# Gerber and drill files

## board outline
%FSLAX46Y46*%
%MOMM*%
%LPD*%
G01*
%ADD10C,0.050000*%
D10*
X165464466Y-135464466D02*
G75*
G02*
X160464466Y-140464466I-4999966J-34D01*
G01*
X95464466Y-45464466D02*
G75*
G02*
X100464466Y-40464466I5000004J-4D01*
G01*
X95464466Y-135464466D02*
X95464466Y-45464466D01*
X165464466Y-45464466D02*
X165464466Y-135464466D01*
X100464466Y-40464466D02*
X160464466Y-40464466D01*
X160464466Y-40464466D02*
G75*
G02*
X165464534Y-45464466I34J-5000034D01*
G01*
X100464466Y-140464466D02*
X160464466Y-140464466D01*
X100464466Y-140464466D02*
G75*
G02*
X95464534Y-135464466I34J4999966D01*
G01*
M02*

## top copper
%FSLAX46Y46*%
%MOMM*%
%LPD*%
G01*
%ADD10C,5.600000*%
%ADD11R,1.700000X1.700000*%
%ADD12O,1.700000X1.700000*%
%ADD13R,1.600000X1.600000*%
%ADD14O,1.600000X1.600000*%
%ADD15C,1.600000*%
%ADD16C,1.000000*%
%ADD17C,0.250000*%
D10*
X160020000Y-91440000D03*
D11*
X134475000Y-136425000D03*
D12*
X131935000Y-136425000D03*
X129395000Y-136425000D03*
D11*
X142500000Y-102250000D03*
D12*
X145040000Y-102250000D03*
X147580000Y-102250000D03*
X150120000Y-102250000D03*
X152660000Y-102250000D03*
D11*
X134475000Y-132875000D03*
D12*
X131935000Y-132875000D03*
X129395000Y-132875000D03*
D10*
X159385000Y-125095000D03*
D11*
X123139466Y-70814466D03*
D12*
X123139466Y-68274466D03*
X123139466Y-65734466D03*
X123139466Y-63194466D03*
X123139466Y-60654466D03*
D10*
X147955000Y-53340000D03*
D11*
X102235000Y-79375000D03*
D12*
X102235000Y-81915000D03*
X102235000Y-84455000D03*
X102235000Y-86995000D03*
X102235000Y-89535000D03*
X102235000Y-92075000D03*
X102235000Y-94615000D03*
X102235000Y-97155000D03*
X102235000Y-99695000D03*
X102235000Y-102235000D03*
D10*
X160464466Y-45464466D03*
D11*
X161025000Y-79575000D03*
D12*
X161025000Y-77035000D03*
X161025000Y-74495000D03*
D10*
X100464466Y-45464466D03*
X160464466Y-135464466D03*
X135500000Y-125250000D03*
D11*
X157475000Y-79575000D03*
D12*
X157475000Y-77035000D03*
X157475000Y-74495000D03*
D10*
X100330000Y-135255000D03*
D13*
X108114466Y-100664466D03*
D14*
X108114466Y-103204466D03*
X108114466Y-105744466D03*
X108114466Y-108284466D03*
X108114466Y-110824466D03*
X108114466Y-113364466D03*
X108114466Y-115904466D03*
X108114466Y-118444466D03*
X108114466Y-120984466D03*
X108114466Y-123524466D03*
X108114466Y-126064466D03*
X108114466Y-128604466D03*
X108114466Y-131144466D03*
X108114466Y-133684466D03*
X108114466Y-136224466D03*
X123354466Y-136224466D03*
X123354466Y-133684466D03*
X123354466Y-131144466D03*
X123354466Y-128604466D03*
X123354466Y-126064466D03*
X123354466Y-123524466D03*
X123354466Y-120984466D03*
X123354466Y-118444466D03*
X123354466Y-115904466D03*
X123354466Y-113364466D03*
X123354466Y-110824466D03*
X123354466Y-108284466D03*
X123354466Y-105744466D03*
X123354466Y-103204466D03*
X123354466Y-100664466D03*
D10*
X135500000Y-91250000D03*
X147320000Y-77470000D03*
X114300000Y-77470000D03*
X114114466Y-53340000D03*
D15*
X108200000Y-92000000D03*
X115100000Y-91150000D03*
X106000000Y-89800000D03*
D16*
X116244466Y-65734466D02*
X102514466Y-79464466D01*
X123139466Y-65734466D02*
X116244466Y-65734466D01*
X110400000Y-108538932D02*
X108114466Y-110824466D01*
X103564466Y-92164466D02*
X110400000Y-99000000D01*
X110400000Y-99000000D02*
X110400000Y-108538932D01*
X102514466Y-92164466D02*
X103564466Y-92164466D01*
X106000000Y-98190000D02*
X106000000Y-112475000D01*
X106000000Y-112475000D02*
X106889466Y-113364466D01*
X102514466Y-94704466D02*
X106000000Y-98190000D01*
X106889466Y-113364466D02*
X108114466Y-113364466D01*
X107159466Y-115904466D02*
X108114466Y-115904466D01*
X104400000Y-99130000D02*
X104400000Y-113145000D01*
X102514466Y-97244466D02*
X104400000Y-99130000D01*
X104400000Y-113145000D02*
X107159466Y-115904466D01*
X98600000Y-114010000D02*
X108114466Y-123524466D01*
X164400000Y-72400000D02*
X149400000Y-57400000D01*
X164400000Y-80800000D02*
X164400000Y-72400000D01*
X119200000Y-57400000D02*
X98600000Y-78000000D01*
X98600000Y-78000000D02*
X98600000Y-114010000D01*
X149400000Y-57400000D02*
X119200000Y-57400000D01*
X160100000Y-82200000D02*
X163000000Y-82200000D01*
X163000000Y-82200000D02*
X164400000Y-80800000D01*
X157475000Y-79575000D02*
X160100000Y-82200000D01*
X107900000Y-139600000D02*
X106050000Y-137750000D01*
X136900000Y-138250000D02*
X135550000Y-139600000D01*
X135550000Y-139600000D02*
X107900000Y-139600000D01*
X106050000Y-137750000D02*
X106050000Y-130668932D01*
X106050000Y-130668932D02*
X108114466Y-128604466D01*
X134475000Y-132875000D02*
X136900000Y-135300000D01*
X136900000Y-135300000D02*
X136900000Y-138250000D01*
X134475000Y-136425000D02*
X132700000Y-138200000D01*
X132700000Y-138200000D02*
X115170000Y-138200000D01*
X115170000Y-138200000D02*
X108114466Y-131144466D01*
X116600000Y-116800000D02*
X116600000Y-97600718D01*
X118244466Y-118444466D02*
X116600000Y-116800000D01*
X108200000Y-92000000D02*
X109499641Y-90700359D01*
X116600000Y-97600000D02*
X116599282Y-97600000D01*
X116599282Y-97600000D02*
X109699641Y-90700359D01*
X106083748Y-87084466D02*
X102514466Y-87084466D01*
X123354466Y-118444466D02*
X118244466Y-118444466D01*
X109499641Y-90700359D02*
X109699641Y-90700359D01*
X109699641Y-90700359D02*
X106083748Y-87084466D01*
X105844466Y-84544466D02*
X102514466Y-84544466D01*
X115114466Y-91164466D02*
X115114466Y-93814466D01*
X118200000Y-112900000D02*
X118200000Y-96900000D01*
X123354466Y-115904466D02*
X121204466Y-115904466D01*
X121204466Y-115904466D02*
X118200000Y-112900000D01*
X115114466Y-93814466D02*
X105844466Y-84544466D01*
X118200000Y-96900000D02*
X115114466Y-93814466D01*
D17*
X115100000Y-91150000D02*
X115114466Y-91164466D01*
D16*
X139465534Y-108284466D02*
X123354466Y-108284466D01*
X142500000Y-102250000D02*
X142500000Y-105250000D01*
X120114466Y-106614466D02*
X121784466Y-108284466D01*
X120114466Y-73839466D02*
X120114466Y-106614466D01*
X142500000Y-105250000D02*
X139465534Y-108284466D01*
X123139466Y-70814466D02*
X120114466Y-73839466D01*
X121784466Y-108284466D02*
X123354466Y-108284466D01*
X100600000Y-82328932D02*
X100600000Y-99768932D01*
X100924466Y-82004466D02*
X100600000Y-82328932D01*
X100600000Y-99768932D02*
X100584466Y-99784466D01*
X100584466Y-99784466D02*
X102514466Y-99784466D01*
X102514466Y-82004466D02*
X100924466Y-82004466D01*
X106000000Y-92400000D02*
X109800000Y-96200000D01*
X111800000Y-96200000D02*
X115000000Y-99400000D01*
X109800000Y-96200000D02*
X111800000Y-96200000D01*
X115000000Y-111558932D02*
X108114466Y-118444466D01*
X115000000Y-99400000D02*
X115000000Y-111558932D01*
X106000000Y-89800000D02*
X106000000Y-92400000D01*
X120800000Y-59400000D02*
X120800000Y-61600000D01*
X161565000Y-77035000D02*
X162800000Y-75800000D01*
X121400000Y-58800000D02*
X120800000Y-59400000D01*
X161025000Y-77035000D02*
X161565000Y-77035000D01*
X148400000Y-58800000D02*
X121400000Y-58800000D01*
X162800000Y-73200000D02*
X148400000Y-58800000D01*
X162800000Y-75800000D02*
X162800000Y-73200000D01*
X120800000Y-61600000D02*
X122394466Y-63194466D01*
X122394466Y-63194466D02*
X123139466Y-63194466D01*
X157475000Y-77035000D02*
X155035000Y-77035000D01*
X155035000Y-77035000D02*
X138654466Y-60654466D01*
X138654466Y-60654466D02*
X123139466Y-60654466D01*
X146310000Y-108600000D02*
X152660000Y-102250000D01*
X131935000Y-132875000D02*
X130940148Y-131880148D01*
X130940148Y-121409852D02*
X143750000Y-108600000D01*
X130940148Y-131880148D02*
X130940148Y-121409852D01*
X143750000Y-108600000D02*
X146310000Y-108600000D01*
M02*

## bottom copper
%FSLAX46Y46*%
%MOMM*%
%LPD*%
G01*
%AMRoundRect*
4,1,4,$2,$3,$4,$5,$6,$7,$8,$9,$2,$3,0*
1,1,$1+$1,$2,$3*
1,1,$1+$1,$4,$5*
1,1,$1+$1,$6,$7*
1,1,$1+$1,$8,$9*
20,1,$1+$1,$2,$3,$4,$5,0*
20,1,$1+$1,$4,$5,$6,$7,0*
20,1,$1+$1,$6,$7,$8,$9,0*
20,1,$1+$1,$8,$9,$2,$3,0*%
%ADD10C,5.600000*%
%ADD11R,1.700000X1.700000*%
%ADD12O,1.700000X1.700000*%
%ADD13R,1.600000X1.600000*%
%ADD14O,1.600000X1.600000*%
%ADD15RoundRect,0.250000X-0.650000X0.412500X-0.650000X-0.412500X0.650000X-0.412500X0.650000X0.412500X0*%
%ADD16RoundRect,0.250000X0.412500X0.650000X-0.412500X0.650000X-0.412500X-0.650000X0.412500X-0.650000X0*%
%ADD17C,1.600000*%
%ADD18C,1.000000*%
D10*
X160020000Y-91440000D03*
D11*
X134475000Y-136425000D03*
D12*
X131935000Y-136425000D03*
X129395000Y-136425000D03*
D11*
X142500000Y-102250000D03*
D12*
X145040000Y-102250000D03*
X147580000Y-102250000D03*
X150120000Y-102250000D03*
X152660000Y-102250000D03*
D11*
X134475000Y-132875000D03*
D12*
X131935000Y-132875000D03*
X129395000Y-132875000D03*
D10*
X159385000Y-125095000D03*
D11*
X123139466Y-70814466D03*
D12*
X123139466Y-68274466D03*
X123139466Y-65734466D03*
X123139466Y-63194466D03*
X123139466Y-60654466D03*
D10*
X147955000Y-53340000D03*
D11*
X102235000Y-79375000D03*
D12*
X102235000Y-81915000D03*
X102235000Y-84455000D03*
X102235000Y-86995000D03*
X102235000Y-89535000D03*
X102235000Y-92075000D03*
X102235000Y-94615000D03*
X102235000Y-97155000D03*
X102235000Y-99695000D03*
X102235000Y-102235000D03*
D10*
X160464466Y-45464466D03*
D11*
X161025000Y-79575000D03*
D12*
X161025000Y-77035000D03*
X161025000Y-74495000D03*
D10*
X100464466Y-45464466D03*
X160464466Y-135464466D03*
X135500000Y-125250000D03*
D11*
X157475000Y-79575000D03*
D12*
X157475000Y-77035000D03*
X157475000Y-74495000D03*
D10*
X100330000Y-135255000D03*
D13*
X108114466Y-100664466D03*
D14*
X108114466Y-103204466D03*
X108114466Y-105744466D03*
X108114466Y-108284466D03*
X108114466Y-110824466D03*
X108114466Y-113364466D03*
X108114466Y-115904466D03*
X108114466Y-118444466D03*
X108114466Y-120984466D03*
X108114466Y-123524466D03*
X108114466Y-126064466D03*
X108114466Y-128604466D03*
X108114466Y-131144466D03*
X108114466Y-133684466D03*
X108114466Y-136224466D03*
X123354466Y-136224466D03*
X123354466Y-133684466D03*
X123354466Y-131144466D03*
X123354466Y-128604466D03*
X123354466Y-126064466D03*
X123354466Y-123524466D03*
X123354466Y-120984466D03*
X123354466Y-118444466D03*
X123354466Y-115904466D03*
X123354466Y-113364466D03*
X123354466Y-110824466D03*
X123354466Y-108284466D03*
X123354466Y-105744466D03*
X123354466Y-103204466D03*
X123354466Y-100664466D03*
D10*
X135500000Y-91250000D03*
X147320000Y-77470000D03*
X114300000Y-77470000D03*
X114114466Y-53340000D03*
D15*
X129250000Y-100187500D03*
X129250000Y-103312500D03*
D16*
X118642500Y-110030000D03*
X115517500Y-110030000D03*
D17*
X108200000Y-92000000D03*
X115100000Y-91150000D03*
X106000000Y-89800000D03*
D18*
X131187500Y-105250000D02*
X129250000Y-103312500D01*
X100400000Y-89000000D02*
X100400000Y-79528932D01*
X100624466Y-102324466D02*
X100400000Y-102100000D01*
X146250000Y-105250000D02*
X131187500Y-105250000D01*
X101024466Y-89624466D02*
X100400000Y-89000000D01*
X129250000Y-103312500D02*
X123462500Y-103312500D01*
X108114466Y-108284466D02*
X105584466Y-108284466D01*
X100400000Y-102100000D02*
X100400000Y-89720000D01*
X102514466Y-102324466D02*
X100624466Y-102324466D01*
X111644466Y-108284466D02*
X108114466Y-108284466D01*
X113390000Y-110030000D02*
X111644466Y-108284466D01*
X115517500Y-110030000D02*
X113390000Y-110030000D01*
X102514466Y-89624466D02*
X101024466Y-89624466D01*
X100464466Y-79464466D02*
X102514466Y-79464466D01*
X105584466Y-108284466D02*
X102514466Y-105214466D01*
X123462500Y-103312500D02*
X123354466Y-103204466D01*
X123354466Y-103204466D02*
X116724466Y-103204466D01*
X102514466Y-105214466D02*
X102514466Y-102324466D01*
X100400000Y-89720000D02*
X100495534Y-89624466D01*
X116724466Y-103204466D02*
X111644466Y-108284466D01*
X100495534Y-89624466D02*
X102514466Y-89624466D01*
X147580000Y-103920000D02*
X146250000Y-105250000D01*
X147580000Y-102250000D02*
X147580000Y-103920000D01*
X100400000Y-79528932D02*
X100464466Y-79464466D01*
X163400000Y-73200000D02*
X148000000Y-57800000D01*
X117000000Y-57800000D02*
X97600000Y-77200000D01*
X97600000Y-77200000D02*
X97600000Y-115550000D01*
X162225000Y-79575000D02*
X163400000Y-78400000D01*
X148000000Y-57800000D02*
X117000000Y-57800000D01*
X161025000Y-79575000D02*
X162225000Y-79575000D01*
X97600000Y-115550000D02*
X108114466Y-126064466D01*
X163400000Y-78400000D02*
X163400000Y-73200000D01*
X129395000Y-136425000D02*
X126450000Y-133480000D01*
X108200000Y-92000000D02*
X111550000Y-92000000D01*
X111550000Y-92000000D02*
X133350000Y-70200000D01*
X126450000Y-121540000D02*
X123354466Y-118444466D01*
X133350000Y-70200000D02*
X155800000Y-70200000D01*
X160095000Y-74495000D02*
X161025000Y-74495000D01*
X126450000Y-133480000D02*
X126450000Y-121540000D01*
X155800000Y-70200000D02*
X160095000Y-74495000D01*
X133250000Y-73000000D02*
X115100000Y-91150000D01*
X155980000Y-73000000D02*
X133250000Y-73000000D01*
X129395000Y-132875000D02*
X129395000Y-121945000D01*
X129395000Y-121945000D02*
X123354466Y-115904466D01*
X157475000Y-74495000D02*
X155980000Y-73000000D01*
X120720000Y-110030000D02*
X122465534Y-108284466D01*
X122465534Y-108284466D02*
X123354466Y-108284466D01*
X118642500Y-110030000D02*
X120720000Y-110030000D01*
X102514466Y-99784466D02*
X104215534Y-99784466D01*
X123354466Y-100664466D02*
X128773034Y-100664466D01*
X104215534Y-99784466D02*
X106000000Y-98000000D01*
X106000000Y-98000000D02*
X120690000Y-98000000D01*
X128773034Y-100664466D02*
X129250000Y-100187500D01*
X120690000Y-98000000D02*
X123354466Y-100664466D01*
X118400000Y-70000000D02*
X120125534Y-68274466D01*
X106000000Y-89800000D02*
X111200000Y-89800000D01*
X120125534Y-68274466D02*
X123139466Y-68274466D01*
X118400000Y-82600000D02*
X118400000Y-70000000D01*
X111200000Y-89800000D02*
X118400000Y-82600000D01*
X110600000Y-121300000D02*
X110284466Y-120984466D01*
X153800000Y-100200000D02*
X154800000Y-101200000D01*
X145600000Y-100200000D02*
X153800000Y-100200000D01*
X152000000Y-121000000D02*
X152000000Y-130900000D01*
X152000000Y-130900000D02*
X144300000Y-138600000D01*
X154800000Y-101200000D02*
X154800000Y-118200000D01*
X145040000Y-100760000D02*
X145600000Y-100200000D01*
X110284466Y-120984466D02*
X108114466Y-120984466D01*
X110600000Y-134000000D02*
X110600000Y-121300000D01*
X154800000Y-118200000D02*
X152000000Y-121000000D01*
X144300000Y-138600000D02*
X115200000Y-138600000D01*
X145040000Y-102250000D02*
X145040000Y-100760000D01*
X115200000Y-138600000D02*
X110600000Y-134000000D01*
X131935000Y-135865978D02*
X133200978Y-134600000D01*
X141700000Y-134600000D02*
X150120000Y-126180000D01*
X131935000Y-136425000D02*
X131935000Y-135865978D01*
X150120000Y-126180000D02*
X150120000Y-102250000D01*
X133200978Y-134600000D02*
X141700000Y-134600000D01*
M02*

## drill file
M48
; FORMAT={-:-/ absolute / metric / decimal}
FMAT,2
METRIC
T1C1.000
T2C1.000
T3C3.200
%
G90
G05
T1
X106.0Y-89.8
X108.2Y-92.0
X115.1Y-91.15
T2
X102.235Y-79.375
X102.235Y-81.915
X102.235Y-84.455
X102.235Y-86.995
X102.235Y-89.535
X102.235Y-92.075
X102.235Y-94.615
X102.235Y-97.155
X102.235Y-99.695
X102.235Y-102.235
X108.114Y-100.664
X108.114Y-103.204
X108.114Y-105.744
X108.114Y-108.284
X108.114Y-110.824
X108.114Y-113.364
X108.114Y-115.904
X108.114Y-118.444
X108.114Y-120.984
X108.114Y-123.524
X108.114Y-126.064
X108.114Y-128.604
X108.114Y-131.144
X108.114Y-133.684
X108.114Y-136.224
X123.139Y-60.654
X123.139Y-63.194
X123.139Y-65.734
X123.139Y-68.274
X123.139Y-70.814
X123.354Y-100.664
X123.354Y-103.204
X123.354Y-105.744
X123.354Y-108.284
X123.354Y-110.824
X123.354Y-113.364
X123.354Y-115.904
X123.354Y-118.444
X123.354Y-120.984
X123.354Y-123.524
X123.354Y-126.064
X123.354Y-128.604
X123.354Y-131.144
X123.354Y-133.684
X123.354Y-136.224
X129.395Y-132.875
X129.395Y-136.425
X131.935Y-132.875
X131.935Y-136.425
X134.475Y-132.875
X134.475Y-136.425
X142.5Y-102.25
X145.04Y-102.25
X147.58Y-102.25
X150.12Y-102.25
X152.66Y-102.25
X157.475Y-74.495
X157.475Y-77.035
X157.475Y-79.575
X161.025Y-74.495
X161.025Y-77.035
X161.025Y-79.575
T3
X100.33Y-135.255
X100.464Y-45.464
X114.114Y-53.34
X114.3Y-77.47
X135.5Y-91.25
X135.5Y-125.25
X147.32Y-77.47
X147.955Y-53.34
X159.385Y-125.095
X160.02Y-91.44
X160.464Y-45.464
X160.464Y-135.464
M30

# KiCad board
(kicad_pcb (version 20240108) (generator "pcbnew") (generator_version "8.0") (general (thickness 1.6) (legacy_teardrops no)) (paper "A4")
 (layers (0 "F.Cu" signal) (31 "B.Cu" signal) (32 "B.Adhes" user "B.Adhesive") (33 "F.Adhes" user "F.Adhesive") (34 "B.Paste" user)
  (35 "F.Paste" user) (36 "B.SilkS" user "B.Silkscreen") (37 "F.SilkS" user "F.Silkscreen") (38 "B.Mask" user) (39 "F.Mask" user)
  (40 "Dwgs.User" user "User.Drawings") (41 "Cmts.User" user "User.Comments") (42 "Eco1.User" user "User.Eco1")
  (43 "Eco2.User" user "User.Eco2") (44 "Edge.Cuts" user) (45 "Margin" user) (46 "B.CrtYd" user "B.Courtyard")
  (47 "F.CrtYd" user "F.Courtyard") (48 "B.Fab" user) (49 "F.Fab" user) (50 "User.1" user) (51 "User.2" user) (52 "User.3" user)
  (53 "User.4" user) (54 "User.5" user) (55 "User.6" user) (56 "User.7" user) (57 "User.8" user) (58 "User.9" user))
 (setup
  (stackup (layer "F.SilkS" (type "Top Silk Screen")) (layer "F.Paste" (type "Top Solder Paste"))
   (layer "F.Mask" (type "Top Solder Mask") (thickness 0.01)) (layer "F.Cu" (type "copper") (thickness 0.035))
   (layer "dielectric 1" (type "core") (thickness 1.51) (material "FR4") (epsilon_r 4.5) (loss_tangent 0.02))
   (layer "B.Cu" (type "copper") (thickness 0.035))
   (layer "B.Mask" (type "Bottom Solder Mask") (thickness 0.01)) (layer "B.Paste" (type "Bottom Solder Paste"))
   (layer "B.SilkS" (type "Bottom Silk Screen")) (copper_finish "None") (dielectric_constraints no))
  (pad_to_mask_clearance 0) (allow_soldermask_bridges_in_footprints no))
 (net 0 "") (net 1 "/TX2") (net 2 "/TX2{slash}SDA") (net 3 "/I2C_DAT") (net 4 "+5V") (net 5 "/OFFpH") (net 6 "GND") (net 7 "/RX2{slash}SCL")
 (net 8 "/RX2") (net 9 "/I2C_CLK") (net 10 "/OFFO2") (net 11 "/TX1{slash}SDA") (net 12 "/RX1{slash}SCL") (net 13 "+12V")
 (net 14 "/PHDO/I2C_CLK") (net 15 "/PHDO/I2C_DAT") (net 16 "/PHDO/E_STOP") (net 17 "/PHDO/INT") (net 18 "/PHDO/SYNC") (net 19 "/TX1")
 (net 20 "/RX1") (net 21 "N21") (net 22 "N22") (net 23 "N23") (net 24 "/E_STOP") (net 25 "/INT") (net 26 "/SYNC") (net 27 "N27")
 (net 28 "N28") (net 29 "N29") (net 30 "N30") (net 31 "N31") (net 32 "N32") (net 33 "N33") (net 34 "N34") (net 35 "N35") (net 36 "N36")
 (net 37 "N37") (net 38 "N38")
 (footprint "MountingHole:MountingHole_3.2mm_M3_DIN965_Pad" (layer "F.Cu") (at 160.02 91.44)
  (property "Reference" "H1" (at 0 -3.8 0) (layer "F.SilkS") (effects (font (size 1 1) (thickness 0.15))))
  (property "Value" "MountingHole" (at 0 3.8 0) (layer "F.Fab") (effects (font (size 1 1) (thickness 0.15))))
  (pad "1" thru_hole circle (at 0 0) (size 5.6 5.6) (drill 3.2) (layers "*.Cu" "*.Mask") (remove_unused_layers no)))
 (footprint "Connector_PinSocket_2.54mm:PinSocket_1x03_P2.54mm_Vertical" (layer "F.Cu") (at 134.475 136.425 -90)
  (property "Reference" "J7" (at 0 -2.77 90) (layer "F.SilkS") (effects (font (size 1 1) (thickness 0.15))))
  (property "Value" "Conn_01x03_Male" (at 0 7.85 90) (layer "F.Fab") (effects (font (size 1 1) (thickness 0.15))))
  (pad "1" thru_hole rect (at 0 0 270) (size 1.7 1.7) (drill 1) (layers "*.Cu" "*.Mask") (remove_unused_layers no) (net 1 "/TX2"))
  (pad "2" thru_hole oval (at 0 2.54 270) (size 1.7 1.7) (drill 1) (layers "*.Cu" "*.Mask") (remove_unused_layers no)
   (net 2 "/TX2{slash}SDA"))
  (pad "3" thru_hole oval (at 0 5.08 270) (size 1.7 1.7) (drill 1) (layers "*.Cu" "*.Mask") (remove_unused_layers no) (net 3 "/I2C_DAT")))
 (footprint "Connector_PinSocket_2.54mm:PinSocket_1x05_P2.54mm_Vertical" (layer "F.Cu") (at 142.5 102.25 90)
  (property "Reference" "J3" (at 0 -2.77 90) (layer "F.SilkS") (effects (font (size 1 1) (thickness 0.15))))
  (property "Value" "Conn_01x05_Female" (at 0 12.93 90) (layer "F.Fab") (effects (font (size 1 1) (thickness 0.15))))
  (pad "1" thru_hole rect (at 0 0 90) (size 1.7 1.7) (drill 1) (layers "*.Cu" "*.Mask") (remove_unused_layers no) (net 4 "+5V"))
  (pad "2" thru_hole oval (at 0 2.54 90) (size 1.7 1.7) (drill 1) (layers "*.Cu" "*.Mask") (remove_unused_layers no) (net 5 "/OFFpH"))
  (pad "3" thru_hole oval (at 0 5.08 90) (size 1.7 1.7) (drill 1) (layers "*.Cu" "*.Mask") (remove_unused_layers no) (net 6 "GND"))
  (pad "4" thru_hole oval (at 0 7.62 90) (size 1.7 1.7) (drill 1) (layers "*.Cu" "*.Mask") (remove_unused_layers no)
   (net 2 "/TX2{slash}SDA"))
  (pad "5" thru_hole oval (at 0 10.16 90) (size 1.7 1.7) (drill 1) (layers "*.Cu" "*.Mask") (remove_unused_layers no)
   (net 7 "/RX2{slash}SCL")))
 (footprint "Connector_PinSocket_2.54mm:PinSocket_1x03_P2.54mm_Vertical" (layer "F.Cu") (at 134.475 132.875 -90)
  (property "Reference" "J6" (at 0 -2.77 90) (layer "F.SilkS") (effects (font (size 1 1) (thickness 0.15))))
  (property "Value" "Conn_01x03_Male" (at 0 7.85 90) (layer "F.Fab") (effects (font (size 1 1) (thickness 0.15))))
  (pad "1" thru_hole rect (at 0 0 270) (size 1.7 1.7) (drill 1) (layers "*.Cu" "*.Mask") (remove_unused_layers no) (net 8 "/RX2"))
  (pad "2" thru_hole oval (at 0 2.54 270) (size 1.7 1.7) (drill 1) (layers "*.Cu" "*.Mask") (remove_unused_layers no)
   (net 7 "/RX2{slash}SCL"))
  (pad "3" thru_hole oval (at 0 5.08 270) (size 1.7 1.7) (drill 1) (layers "*.Cu" "*.Mask") (remove_unused_layers no) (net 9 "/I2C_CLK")))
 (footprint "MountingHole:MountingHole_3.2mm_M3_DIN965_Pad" (layer "F.Cu") (at 159.385 125.095)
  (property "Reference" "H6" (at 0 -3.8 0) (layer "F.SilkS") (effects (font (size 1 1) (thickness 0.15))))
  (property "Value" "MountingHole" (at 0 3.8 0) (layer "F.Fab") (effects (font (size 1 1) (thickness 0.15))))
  (pad "1" thru_hole circle (at 0 0) (size 5.6 5.6) (drill 3.2) (layers "*.Cu" "*.Mask") (remove_unused_layers no)))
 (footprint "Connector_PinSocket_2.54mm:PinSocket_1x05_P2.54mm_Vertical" (layer "F.Cu") (at 123.139466 70.814466 180)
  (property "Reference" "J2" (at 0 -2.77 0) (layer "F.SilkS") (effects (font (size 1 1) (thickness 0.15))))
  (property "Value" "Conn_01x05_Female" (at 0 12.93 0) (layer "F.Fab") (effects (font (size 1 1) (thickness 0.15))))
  (pad "1" thru_hole rect (at 0 0 180) (size 1.7 1.7) (drill 1) (layers "*.Cu" "*.Mask") (remove_unused_layers no) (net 4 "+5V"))
  (pad "2" thru_hole oval (at 0 2.54 180) (size 1.7 1.7) (drill 1) (layers "*.Cu" "*.Mask") (remove_unused_layers no) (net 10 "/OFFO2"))
  (pad "3" thru_hole oval (at 0 5.08 180) (size 1.7 1.7) (drill 1) (layers "*.Cu" "*.Mask") (remove_unused_layers no) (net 6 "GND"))
  (pad "4" thru_hole oval (at 0 7.62 180) (size 1.7 1.7) (drill 1) (layers "*.Cu" "*.Mask") (remove_unused_layers no)
   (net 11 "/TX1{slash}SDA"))
  (pad "5" thru_hole oval (at 0 10.16 180) (size 1.7 1.7) (drill 1) (layers "*.Cu" "*.Mask") (remove_unused_layers no)
   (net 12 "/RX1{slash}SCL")))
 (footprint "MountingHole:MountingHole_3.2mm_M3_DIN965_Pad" (layer "F.Cu") (at 147.955 53.34)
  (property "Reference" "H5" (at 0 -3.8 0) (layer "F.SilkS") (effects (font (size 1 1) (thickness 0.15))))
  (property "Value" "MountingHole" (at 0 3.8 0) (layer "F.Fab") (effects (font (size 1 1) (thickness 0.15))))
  (pad "1" thru_hole circle (at 0 0) (size 5.6 5.6) (drill 3.2) (layers "*.Cu" "*.Mask") (remove_unused_layers no)))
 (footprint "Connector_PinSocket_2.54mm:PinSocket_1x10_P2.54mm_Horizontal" (layer "F.Cu") (at 102.235 79.375)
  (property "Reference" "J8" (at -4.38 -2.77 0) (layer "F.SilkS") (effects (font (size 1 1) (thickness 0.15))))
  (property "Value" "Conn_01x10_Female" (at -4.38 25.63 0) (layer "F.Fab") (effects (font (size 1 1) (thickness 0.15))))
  (pad "1" thru_hole rect (at 0 0) (size 1.7 1.7) (drill 1) (layers "*.Cu" "*.Mask") (remove_unused_layers no) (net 6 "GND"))
  (pad "2" thru_hole oval (at 0 2.54) (size 1.7 1.7) (drill 1) (layers "*.Cu" "*.Mask") (remove_unused_layers no) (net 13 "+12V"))
  (pad "3" thru_hole oval (at 0 5.08) (size 1.7 1.7) (drill 1) (layers "*.Cu" "*.Mask") (remove_unused_layers no) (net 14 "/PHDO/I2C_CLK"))
  (pad "4" thru_hole oval (at 0 7.62) (size 1.7 1.7) (drill 1) (layers "*.Cu" "*.Mask") (remove_unused_layers no) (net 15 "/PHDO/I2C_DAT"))
  (pad "5" thru_hole oval (at 0 10.16) (size 1.7 1.7) (drill 1) (layers "*.Cu" "*.Mask") (remove_unused_layers no) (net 6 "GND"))
  (pad "6" thru_hole oval (at 0 12.7) (size 1.7 1.7) (drill 1) (layers "*.Cu" "*.Mask") (remove_unused_layers no) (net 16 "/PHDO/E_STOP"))
  (pad "7" thru_hole oval (at 0 15.24) (size 1.7 1.7) (drill 1) (layers "*.Cu" "*.Mask") (remove_unused_layers no) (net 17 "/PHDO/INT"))
  (pad "8" thru_hole oval (at 0 17.78) (size 1.7 1.7) (drill 1) (layers "*.Cu" "*.Mask") (remove_unused_layers no) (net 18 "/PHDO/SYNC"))
  (pad "9" thru_hole oval (at 0 20.32) (size 1.7 1.7) (drill 1) (layers "*.Cu" "*.Mask") (remove_unused_layers no) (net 13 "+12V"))
  (pad "10" thru_hole oval (at 0 22.86) (size 1.7 1.7) (drill 1) (layers "*.Cu" "*.Mask") (remove_unused_layers no) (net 6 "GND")))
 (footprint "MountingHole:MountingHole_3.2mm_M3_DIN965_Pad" (layer "F.Cu") (at 160.464466 45.464466)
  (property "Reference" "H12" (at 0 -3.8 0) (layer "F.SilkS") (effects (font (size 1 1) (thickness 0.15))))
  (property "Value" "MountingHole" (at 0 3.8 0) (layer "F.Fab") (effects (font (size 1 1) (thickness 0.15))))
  (pad "1" thru_hole circle (at 0 0) (size 5.6 5.6) (drill 3.2) (layers "*.Cu" "*.Mask") (remove_unused_layers no)))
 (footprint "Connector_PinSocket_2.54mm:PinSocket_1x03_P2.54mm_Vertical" (layer "F.Cu") (at 161.025 79.575 180)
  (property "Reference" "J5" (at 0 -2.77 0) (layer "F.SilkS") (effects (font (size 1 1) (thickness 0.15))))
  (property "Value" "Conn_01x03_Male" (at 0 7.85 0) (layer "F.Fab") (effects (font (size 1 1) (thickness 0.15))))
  (pad "1" thru_hole rect (at 0 0 180) (size 1.7 1.7) (drill 1) (layers "*.Cu" "*.Mask") (remove_unused_layers no) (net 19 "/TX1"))
  (pad "2" thru_hole oval (at 0 2.54 180) (size 1.7 1.7) (drill 1) (layers "*.Cu" "*.Mask") (remove_unused_layers no)
   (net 11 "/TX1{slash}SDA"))
  (pad "3" thru_hole oval (at 0 5.08 180) (size 1.7 1.7) (drill 1) (layers "*.Cu" "*.Mask") (remove_unused_layers no) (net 3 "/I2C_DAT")))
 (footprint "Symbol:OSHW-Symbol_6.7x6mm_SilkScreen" (layer "F.Cu") (at 109.515 44.979 180)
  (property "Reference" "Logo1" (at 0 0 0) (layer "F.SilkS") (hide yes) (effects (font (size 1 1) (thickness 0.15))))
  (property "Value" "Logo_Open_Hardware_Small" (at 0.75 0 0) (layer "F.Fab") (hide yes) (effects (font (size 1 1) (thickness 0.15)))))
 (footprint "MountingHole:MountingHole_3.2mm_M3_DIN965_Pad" (layer "F.Cu") (at 100.464466 45.464466)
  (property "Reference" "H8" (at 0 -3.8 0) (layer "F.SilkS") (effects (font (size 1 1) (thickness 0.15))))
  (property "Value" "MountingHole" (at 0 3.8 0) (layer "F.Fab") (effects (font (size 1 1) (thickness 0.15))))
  (pad "1" thru_hole circle (at 0 0) (size 5.6 5.6) (drill 3.2) (layers "*.Cu" "*.Mask") (remove_unused_layers no)))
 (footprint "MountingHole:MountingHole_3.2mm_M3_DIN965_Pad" (layer "F.Cu") (at 160.464466 135.464466)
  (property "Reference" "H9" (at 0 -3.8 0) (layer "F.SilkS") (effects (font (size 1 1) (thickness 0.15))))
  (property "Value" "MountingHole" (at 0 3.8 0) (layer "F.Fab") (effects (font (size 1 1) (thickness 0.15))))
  (pad "1" thru_hole circle (at 0 0) (size 5.6 5.6) (drill 3.2) (layers "*.Cu" "*.Mask") (remove_unused_layers no)))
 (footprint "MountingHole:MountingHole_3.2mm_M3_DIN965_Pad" (layer "F.Cu") (at 135.5 125.25 90)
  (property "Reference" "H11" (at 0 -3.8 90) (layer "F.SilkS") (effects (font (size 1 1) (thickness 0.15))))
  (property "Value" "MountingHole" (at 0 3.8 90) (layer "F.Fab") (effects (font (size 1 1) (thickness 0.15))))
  (pad "1" thru_hole circle (at 0 0 90) (size 5.6 5.6) (drill 3.2) (layers "*.Cu" "*.Mask") (remove_unused_layers no)))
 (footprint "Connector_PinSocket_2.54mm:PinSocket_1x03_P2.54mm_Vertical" (layer "F.Cu") (at 157.475 79.575 180)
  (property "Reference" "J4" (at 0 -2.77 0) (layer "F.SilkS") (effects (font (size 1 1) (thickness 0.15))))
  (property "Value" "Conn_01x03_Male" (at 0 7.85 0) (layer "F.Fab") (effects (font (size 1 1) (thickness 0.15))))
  (pad "1" thru_hole rect (at 0 0 180) (size 1.7 1.7) (drill 1) (layers "*.Cu" "*.Mask") (remove_unused_layers no) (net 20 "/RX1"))
  (pad "2" thru_hole oval (at 0 2.54 180) (size 1.7 1.7) (drill 1) (layers "*.Cu" "*.Mask") (remove_unused_layers no)
   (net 12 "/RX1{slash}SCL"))
  (pad "3" thru_hole oval (at 0 5.08 180) (size 1.7 1.7) (drill 1) (layers "*.Cu" "*.Mask") (remove_unused_layers no) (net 9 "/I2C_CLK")))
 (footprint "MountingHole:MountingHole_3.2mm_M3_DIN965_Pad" (layer "F.Cu") (at 100.33 135.255)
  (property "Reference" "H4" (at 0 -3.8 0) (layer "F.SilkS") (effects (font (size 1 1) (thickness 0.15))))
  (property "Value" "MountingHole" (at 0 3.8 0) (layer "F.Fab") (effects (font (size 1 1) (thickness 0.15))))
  (pad "1" thru_hole circle (at 0 0) (size 5.6 5.6) (drill 3.2) (layers "*.Cu" "*.Mask") (remove_unused_layers no)))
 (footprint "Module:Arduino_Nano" (layer "F.Cu") (at 108.114466 100.664466)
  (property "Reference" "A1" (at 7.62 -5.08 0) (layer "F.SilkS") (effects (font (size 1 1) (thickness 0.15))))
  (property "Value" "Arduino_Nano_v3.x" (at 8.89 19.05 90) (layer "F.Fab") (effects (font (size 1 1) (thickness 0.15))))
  (pad "1" thru_hole rect (at 0 0) (size 1.6 1.6) (drill 1) (layers "*.Cu" "*.Mask") (remove_unused_layers no) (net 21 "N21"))
  (pad "2" thru_hole oval (at 0 2.54) (size 1.6 1.6) (drill 1) (layers "*.Cu" "*.Mask") (remove_unused_layers no) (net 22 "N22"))
  (pad "3" thru_hole oval (at 0 5.08) (size 1.6 1.6) (drill 1) (layers "*.Cu" "*.Mask") (remove_unused_layers no) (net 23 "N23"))
  (pad "4" thru_hole oval (at 0 7.62) (size 1.6 1.6) (drill 1) (layers "*.Cu" "*.Mask") (remove_unused_layers no) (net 6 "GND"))
  (pad "5" thru_hole oval (at 0 10.16) (size 1.6 1.6) (drill 1) (layers "*.Cu" "*.Mask") (remove_unused_layers no) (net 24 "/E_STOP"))
  (pad "6" thru_hole oval (at 0 12.7) (size 1.6 1.6) (drill 1) (layers "*.Cu" "*.Mask") (remove_unused_layers no) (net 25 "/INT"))
  (pad "7" thru_hole oval (at 0 15.24) (size 1.6 1.6) (drill 1) (layers "*.Cu" "*.Mask") (remove_unused_layers no) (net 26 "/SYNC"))
  (pad "8" thru_hole oval (at 0 17.78) (size 1.6 1.6) (drill 1) (layers "*.Cu" "*.Mask") (remove_unused_layers no) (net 10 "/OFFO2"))
  (pad "9" thru_hole oval (at 0 20.32) (size 1.6 1.6) (drill 1) (layers "*.Cu" "*.Mask") (remove_unused_layers no) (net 5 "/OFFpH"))
  (pad "10" thru_hole oval (at 0 22.86) (size 1.6 1.6) (drill 1) (layers "*.Cu" "*.Mask") (remove_unused_layers no) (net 20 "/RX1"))
  (pad "11" thru_hole oval (at 0 25.4) (size 1.6 1.6) (drill 1) (layers "*.Cu" "*.Mask") (remove_unused_layers no) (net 19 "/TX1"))
  (pad "12" thru_hole oval (at 0 27.94) (size 1.6 1.6) (drill 1) (layers "*.Cu" "*.Mask") (remove_unused_layers no) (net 8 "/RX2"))
  (pad "13" thru_hole oval (at 0 30.48) (size 1.6 1.6) (drill 1) (layers "*.Cu" "*.Mask") (remove_unused_layers no) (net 1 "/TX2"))
  (pad "14" thru_hole oval (at 0 33.02) (size 1.6 1.6) (drill 1) (layers "*.Cu" "*.Mask") (remove_unused_layers no) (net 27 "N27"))
  (pad "15" thru_hole oval (at 0 35.56) (size 1.6 1.6) (drill 1) (layers "*.Cu" "*.Mask") (remove_unused_layers no) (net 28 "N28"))
  (pad "16" thru_hole oval (at 15.24 35.56) (size 1.6 1.6) (drill 1) (layers "*.Cu" "*.Mask") (remove_unused_layers no) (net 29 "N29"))
  (pad "17" thru_hole oval (at 15.24 33.02) (size 1.6 1.6) (drill 1) (layers "*.Cu" "*.Mask") (remove_unused_layers no) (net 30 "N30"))
  (pad "18" thru_hole oval (at 15.24 30.48) (size 1.6 1.6) (drill 1) (layers "*.Cu" "*.Mask") (remove_unused_layers no) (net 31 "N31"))
  (pad "19" thru_hole oval (at 15.24 27.94) (size 1.6 1.6) (drill 1) (layers "*.Cu" "*.Mask") (remove_unused_layers no) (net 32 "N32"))
  (pad "20" thru_hole oval (at 15.24 25.4) (size 1.6 1.6) (drill 1) (layers "*.Cu" "*.Mask") (remove_unused_layers no) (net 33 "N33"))
  (pad "21" thru_hole oval (at 15.24 22.86) (size 1.6 1.6) (drill 1) (layers "*.Cu" "*.Mask") (remove_unused_layers no) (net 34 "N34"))
  (pad "22" thru_hole oval (at 15.24 20.32) (size 1.6 1.6) (drill 1) (layers "*.Cu" "*.Mask") (remove_unused_layers no) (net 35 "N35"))
  (pad "23" thru_hole oval (at 15.24 17.78) (size 1.6 1.6) (drill 1) (layers "*.Cu" "*.Mask") (remove_unused_layers no) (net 3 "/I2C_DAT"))
  (pad "24" thru_hole oval (at 15.24 15.24) (size 1.6 1.6) (drill 1) (layers "*.Cu" "*.Mask") (remove_unused_layers no) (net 9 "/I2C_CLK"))
  (pad "25" thru_hole oval (at 15.24 12.7) (size 1.6 1.6) (drill 1) (layers "*.Cu" "*.Mask") (remove_unused_layers no) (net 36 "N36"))
  (pad "26" thru_hole oval (at 15.24 10.16) (size 1.6 1.6) (drill 1) (layers "*.Cu" "*.Mask") (remove_unused_layers no) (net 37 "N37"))
  (pad "27" thru_hole oval (at 15.24 7.62) (size 1.6 1.6) (drill 1) (layers "*.Cu" "*.Mask") (remove_unused_layers no) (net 4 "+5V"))
  (pad "28" thru_hole oval (at 15.24 5.08) (size 1.6 1.6) (drill 1) (layers "*.Cu" "*.Mask") (remove_unused_layers no) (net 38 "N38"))
  (pad "29" thru_hole oval (at 15.24 2.54) (size 1.6 1.6) (drill 1) (layers "*.Cu" "*.Mask") (remove_unused_layers no) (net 6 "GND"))
  (pad "30" thru_hole oval (at 15.24 0) (size 1.6 1.6) (drill 1) (layers "*.Cu" "*.Mask") (remove_unused_layers no) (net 13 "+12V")))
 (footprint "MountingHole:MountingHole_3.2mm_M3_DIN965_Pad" (layer "F.Cu") (at 135.5 91.25 90)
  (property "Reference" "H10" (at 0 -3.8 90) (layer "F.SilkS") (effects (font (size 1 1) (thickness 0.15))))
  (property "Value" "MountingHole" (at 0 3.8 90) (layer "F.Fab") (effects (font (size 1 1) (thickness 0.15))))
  (pad "1" thru_hole circle (at 0 0 90) (size 5.6 5.6) (drill 3.2) (layers "*.Cu" "*.Mask") (remove_unused_layers no)))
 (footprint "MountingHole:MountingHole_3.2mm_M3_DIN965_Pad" (layer "F.Cu") (at 147.32 77.47)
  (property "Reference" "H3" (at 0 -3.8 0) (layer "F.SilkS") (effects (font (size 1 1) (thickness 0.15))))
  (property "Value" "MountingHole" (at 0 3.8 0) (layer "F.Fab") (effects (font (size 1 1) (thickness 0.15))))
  (pad "1" thru_hole circle (at 0 0) (size 5.6 5.6) (drill 3.2) (layers "*.Cu" "*.Mask") (remove_unused_layers no)))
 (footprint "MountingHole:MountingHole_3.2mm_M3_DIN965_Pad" (layer "F.Cu") (at 114.3 77.47)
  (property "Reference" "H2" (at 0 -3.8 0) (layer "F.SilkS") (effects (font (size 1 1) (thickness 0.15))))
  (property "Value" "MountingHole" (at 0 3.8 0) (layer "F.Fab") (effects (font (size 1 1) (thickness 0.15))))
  (pad "1" thru_hole circle (at 0 0) (size 5.6 5.6) (drill 3.2) (layers "*.Cu" "*.Mask") (remove_unused_layers no)))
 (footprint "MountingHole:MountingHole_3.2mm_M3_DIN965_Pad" (layer "F.Cu") (at 114.114466 53.34)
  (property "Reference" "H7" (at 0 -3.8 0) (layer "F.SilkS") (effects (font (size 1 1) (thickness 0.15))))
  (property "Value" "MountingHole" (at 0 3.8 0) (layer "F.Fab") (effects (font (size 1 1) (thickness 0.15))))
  (pad "1" thru_hole circle (at 0 0) (size 5.6 5.6) (drill 3.2) (layers "*.Cu" "*.Mask") (remove_unused_layers no)))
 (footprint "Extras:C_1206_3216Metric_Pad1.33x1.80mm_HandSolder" (layer "B.Cu") (at 129.25 101.75 -90)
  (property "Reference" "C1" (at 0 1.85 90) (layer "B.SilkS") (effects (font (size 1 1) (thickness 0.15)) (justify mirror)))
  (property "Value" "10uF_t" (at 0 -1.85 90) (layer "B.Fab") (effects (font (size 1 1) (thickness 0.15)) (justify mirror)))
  (pad "1" smd roundrect (at -1.5625 0 270) (size 1.325 1.8) (layers "B.Cu" "B.Paste" "B.Mask") (roundrect_rratio 0.1886792453)
   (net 13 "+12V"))
  (pad "2" smd roundrect (at 1.5625 0 270) (size 1.325 1.8) (layers "B.Cu" "B.Paste" "B.Mask") (roundrect_rratio 0.1886792453) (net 6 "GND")))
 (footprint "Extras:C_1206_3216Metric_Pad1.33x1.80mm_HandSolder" (layer "B.Cu") (at 117.08 110.03 180)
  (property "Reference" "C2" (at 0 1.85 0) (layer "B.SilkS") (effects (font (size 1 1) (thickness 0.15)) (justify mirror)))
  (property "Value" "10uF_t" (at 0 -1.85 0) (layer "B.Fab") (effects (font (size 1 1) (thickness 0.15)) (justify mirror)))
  (pad "1" smd roundrect (at -1.5625 0 180) (size 1.325 1.8) (layers "B.Cu" "B.Paste" "B.Mask") (roundrect_rratio 0.1886792453)
   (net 4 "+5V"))
  (pad "2" smd roundrect (at 1.5625 0 180) (size 1.325 1.8) (layers "B.Cu" "B.Paste" "B.Mask") (roundrect_rratio 0.1886792453) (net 6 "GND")))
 (gr_arc (start 165.464466 135.464466) (mid 164 139) (end 160.464466 140.464466) (stroke (width 0.05) (type solid)) (layer "Edge.Cuts"))
 (gr_arc (start 95.464466 45.464466) (mid 96.928932 41.928932) (end 100.464466 40.464466) (stroke (width 0.05) (type solid))
  (layer "Edge.Cuts"))
 (gr_line (start 95.464466 135.464466) (end 95.464466 45.464466) (stroke (width 0.05) (type solid)) (layer "Edge.Cuts"))
 (gr_line (start 165.464466 45.464466) (end 165.464466 135.464466) (stroke (width 0.05) (type solid)) (layer "Edge.Cuts"))
 (gr_line (start 100.464466 40.464466) (end 160.464466 40.464466) (stroke (width 0.05) (type solid)) (layer "Edge.Cuts"))
 (gr_arc (start 160.464466 40.464466) (mid 164 41.928932) (end 165.464466 45.464466) (stroke (width 0.05) (type solid)) (layer "Edge.Cuts"))
 (gr_line (start 100.464466 140.464466) (end 160.464466 140.464466) (stroke (width 0.05) (type solid)) (layer "Edge.Cuts"))
 (gr_arc (start 100.464466 140.464466) (mid 96.928932 139) (end 95.464466 135.464466) (stroke (width 0.05) (type solid)) (layer "Edge.Cuts"))
 (segment (start 116.244466 65.734466) (end 102.514466 79.464466) (width 1) (layer "F.Cu") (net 6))
 (segment (start 123.139466 65.734466) (end 116.244466 65.734466) (width 1) (layer "F.Cu") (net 6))
 (segment (start 131.1875 105.25) (end 129.25 103.3125) (width 1) (layer "B.Cu") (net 6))
 (segment (start 100.4 89) (end 100.4 79.528932) (width 1) (layer "B.Cu") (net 6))
 (segment (start 100.624466 102.324466) (end 100.4 102.1) (width 1) (layer "B.Cu") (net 6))
 (segment (start 146.25 105.25) (end 131.1875 105.25) (width 1) (layer "B.Cu") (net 6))
 (segment (start 101.024466 89.624466) (end 100.4 89) (width 1) (layer "B.Cu") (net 6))
 (segment (start 129.25 103.3125) (end 123.4625 103.3125) (width 1) (layer "B.Cu") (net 6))
 (segment (start 108.114466 108.284466) (end 105.584466 108.284466) (width 1) (layer "B.Cu") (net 6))
 (segment (start 100.4 102.1) (end 100.4 89.72) (width 1) (layer "B.Cu") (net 6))
 (segment (start 102.514466 102.324466) (end 100.624466 102.324466) (width 1) (layer "B.Cu") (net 6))
 (segment (start 111.644466 108.284466) (end 108.114466 108.284466) (width 1) (layer "B.Cu") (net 6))
 (segment (start 113.39 110.03) (end 111.644466 108.284466) (width 1) (layer "B.Cu") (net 6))
 (segment (start 115.5175 110.03) (end 113.39 110.03) (width 1) (layer "B.Cu") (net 6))
 (segment (start 102.514466 89.624466) (end 101.024466 89.624466) (width 1) (layer "B.Cu") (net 6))
 (segment (start 100.464466 79.464466) (end 102.514466 79.464466) (width 1) (layer "B.Cu") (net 6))
 (segment (start 105.584466 108.284466) (end 102.514466 105.214466) (width 1) (layer "B.Cu") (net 6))
 (segment (start 123.4625 103.3125) (end 123.354466 103.204466) (width 1) (layer "B.Cu") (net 6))
 (segment (start 123.354466 103.204466) (end 116.724466 103.204466) (width 1) (layer "B.Cu") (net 6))
 (segment (start 102.514466 105.214466) (end 102.514466 102.324466) (width 1) (layer "B.Cu") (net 6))
 (segment (start 100.4 89.72) (end 100.495534 89.624466) (width 1) (layer "B.Cu") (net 6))
 (segment (start 116.724466 103.204466) (end 111.644466 108.284466) (width 1) (layer "B.Cu") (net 6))
 (segment (start 100.495534 89.624466) (end 102.514466 89.624466) (width 1) (layer "B.Cu") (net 6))
 (segment (start 147.58 103.92) (end 146.25 105.25) (width 1) (layer "B.Cu") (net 6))
 (segment (start 147.58 102.25) (end 147.58 103.92) (width 1) (layer "B.Cu") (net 6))
 (segment (start 100.4 79.528932) (end 100.464466 79.464466) (width 1) (layer "B.Cu") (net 6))
 (segment (start 110.4 108.538932) (end 108.114466 110.824466) (width 1) (layer "F.Cu") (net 24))
 (segment (start 103.564466 92.164466) (end 110.4 99) (width 1) (layer "F.Cu") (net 24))
 (segment (start 110.4 99) (end 110.4 108.538932) (width 1) (layer "F.Cu") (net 24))
 (segment (start 102.514466 92.164466) (end 103.564466 92.164466) (width 1) (layer "F.Cu") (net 24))
 (segment (start 106 98.19) (end 106 112.475) (width 1) (layer "F.Cu") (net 25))
 (segment (start 106 112.475) (end 106.889466 113.364466) (width 1) (layer "F.Cu") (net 25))
 (segment (start 102.514466 94.704466) (end 106 98.19) (width 1) (layer "F.Cu") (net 25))
 (segment (start 106.889466 113.364466) (end 108.114466 113.364466) (width 1) (layer "F.Cu") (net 25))
 (segment (start 107.159466 115.904466) (end 108.114466 115.904466) (width 1) (layer "F.Cu") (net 26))
 (segment (start 104.4 99.13) (end 104.4 113.145) (width 1) (layer "F.Cu") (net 26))
 (segment (start 102.514466 97.244466) (end 104.4 99.13) (width 1) (layer "F.Cu") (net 26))
 (segment (start 104.4 113.145) (end 107.159466 115.904466) (width 1) (layer "F.Cu") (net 26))
 (segment (start 98.6 114.01) (end 108.114466 123.524466) (width 1) (layer "F.Cu") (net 20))
 (segment (start 164.4 72.4) (end 149.4 57.4) (width 1) (layer "F.Cu") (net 20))
 (segment (start 164.4 80.8) (end 164.4 72.4) (width 1) (layer "F.Cu") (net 20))
 (segment (start 119.2 57.4) (end 98.6 78) (width 1) (layer "F.Cu") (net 20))
 (segment (start 98.6 78) (end 98.6 114.01) (width 1) (layer "F.Cu") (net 20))
 (segment (start 149.4 57.4) (end 119.2 57.4) (width 1) (layer "F.Cu") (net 20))
 (segment (start 160.1 82.2) (end 163 82.2) (width 1) (layer "F.Cu") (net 20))
 (segment (start 163 82.2) (end 164.4 80.8) (width 1) (layer "F.Cu") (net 20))
 (segment (start 157.475 79.575) (end 160.1 82.2) (width 1) (layer "F.Cu") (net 20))
 (segment (start 163.4 73.2) (end 148 57.8) (width 1) (layer "B.Cu") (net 19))
 (segment (start 117 57.8) (end 97.6 77.2) (width 1) (layer "B.Cu") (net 19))
 (segment (start 97.6 77.2) (end 97.6 115.55) (width 1) (layer "B.Cu") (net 19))
 (segment (start 162.225 79.575) (end 163.4 78.4) (width 1) (layer "B.Cu") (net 19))
 (segment (start 148 57.8) (end 117 57.8) (width 1) (layer "B.Cu") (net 19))
 (segment (start 161.025 79.575) (end 162.225 79.575) (width 1) (layer "B.Cu") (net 19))
 (segment (start 97.6 115.55) (end 108.114466 126.064466) (width 1) (layer "B.Cu") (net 19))
 (segment (start 163.4 78.4) (end 163.4 73.2) (width 1) (layer "B.Cu") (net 19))
 (segment (start 107.9 139.6) (end 106.05 137.75) (width 1) (layer "F.Cu") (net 8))
 (segment (start 136.9 138.25) (end 135.55 139.6) (width 1) (layer "F.Cu") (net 8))
 (segment (start 135.55 139.6) (end 107.9 139.6) (width 1) (layer "F.Cu") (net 8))
 (segment (start 106.05 137.75) (end 106.05 130.668932) (width 1) (layer "F.Cu") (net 8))
 (segment (start 106.05 130.668932) (end 108.114466 128.604466) (width 1) (layer "F.Cu") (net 8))
 (segment (start 134.475 132.875) (end 136.9 135.3) (width 1) (layer "F.Cu") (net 8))
 (segment (start 136.9 135.3) (end 136.9 138.25) (width 1) (layer "F.Cu") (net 8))
 (segment (start 134.475 136.425) (end 132.7 138.2) (width 1) (layer "F.Cu") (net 1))
 (segment (start 132.7 138.2) (end 115.17 138.2) (width 1) (layer "F.Cu") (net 1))
 (segment (start 115.17 138.2) (end 108.114466 131.144466) (width 1) (layer "F.Cu") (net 1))
 (segment (start 116.6 116.8) (end 116.6 97.600718) (width 1) (layer "F.Cu") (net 3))
 (segment (start 118.244466 118.444466) (end 116.6 116.8) (width 1) (layer "F.Cu") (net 3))
 (segment (start 108.2 92) (end 109.499641 90.700359) (width 1) (layer "F.Cu") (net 3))
 (segment (start 116.6 97.6) (end 116.599282 97.6) (width 1) (layer "F.Cu") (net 3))
 (segment (start 116.599282 97.6) (end 109.699641 90.700359) (width 1) (layer "F.Cu") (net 3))
 (segment (start 106.083748 87.084466) (end 102.514466 87.084466) (width 1) (layer "F.Cu") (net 3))
 (segment (start 123.354466 118.444466) (end 118.244466 118.444466) (width 1) (layer "F.Cu") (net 3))
 (segment (start 109.499641 90.700359) (end 109.699641 90.700359) (width 1) (layer "F.Cu") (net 3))
 (segment (start 109.699641 90.700359) (end 106.083748 87.084466) (width 1) (layer "F.Cu") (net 3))
 (via (at 108.2 92) (size 1.6) (drill 1) (layers "F.Cu" "B.Cu") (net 3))
 (segment (start 129.395 136.425) (end 126.45 133.48) (width 1) (layer "B.Cu") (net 3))
 (segment (start 108.2 92) (end 111.55 92) (width 1) (layer "B.Cu") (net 3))
 (segment (start 111.55 92) (end 133.35 70.2) (width 1) (layer "B.Cu") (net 3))
 (segment (start 126.45 121.54) (end 123.354466 118.444466) (width 1) (layer "B.Cu") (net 3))
 (segment (start 133.35 70.2) (end 155.8 70.2) (width 1) (layer "B.Cu") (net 3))
 (segment (start 160.095 74.495) (end 161.025 74.495) (width 1) (layer "B.Cu") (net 3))
 (segment (start 126.45 133.48) (end 126.45 121.54) (width 1) (layer "B.Cu") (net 3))
 (segment (start 155.8 70.2) (end 160.095 74.495) (width 1) (layer "B.Cu") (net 3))
 (segment (start 105.844466 84.544466) (end 102.514466 84.544466) (width 1) (layer "F.Cu") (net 9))
 (segment (start 115.114466 91.164466) (end 115.114466 93.814466) (width 1) (layer "F.Cu") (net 9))
 (segment (start 118.2 112.9) (end 118.2 96.9) (width 1) (layer "F.Cu") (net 9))
 (segment (start 123.354466 115.904466) (end 121.204466 115.904466) (width 1) (layer "F.Cu") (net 9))
 (segment (start 121.204466 115.904466) (end 118.2 112.9) (width 1) (layer "F.Cu") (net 9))
 (segment (start 115.114466 93.814466) (end 105.844466 84.544466) (width 1) (layer "F.Cu") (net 9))
 (segment (start 118.2 96.9) (end 115.114466 93.814466) (width 1) (layer "F.Cu") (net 9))
 (segment (start 115.1 91.15) (end 115.114466 91.164466) (width 0.25) (layer "F.Cu") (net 9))
 (via (at 115.1 91.15) (size 1.6) (drill 1) (layers "F.Cu" "B.Cu") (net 9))
 (segment (start 133.25 73) (end 115.1 91.15) (width 1) (layer "B.Cu") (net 9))
 (segment (start 155.98 73) (end 133.25 73) (width 1) (layer "B.Cu") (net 9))
 (segment (start 129.395 132.875) (end 129.395 121.945) (width 1) (layer "B.Cu") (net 9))
 (segment (start 129.395 121.945) (end 123.354466 115.904466) (width 1) (layer "B.Cu") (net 9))
 (segment (start 157.475 74.495) (end 155.98 73) (width 1) (layer "B.Cu") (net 9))
 (segment (start 139.465534 108.284466) (end 123.354466 108.284466) (width 1) (layer "F.Cu") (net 4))
 (segment (start 142.5 102.25) (end 142.5 105.25) (width 1) (layer "F.Cu") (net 4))
 (segment (start 120.114466 106.614466) (end 121.784466 108.284466) (width 1) (layer "F.Cu") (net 4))
 (segment (start 120.114466 73.839466) (end 120.114466 106.614466) (width 1) (layer "F.Cu") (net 4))
 (segment (start 142.5 105.25) (end 139.465534 108.284466) (width 1) (layer "F.Cu") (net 4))
 (segment (start 123.139466 70.814466) (end 120.114466 73.839466) (width 1) (layer "F.Cu") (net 4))
 (segment (start 121.784466 108.284466) (end 123.354466 108.284466) (width 1) (layer "F.Cu") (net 4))
 (segment (start 120.72 110.03) (end 122.465534 108.284466) (width 1) (layer "B.Cu") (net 4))
 (segment (start 122.465534 108.284466) (end 123.354466 108.284466) (width 1) (layer "B.Cu") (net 4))
 (segment (start 118.6425 110.03) (end 120.72 110.03) (width 1) (layer "B.Cu") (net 4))
 (segment (start 100.6 82.328932) (end 100.6 99.768932) (width 1) (layer "F.Cu") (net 13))
 (segment (start 100.924466 82.004466) (end 100.6 82.328932) (width 1) (layer "F.Cu") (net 13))
 (segment (start 100.6 99.768932) (end 100.584466 99.784466) (width 1) (layer "F.Cu") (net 13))
 (segment (start 100.584466 99.784466) (end 102.514466 99.784466) (width 1) (layer "F.Cu") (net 13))
 (segment (start 102.514466 82.004466) (end 100.924466 82.004466) (width 1) (layer "F.Cu") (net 13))
 (segment (start 102.514466 99.784466) (end 104.215534 99.784466) (width 1) (layer "B.Cu") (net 13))
 (segment (start 123.354466 100.664466) (end 128.773034 100.664466) (width 1) (layer "B.Cu") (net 13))
 (segment (start 104.215534 99.784466) (end 106 98) (width 1) (layer "B.Cu") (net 13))
 (segment (start 106 98) (end 120.69 98) (width 1) (layer "B.Cu") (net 13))
 (segment (start 128.773034 100.664466) (end 129.25 100.1875) (width 1) (layer "B.Cu") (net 13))
 (segment (start 120.69 98) (end 123.354466 100.664466) (width 1) (layer "B.Cu") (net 13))
 (segment (start 106 92.4) (end 109.8 96.2) (width 1) (layer "F.Cu") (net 10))
 (segment (start 111.8 96.2) (end 115 99.4) (width 1) (layer "F.Cu") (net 10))
 (segment (start 109.8 96.2) (end 111.8 96.2) (width 1) (layer "F.Cu") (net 10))
 (segment (start 115 111.558932) (end 108.114466 118.444466) (width 1) (layer "F.Cu") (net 10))
 (segment (start 115 99.4) (end 115 111.558932) (width 1) (layer "F.Cu") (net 10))
 (segment (start 106 89.8) (end 106 92.4) (width 1) (layer "F.Cu") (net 10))
 (via (at 106 89.8) (size 1.6) (drill 1) (layers "F.Cu" "B.Cu") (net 10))
 (segment (start 118.4 70) (end 120.125534 68.274466) (width 1) (layer "B.Cu") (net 10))
 (segment (start 106 89.8) (end 111.2 89.8) (width 1) (layer "B.Cu") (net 10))
 (segment (start 120.125534 68.274466) (end 123.139466 68.274466) (width 1) (layer "B.Cu") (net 10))
 (segment (start 118.4 82.6) (end 118.4 70) (width 1) (layer "B.Cu") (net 10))
 (segment (start 111.2 89.8) (end 118.4 82.6) (width 1) (layer "B.Cu") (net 10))
 (segment (start 110.6 121.3) (end 110.284466 120.984466) (width 1) (layer "B.Cu") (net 5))
 (segment (start 153.8 100.2) (end 154.8 101.2) (width 1) (layer "B.Cu") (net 5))
 (segment (start 145.6 100.2) (end 153.8 100.2) (width 1) (layer "B.Cu") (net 5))
 (segment (start 152 121) (end 152 130.9) (width 1) (layer "B.Cu") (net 5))
 (segment (start 152 130.9) (end 144.3 138.6) (width 1) (layer "B.Cu") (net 5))
 (segment (start 154.8 101.2) (end 154.8 118.2) (width 1) (layer "B.Cu") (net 5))
 (segment (start 145.04 100.76) (end 145.6 100.2) (width 1) (layer "B.Cu") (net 5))
 (segment (start 110.284466 120.984466) (end 108.114466 120.984466) (width 1) (layer "B.Cu") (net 5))
 (segment (start 110.6 134) (end 110.6 121.3) (width 1) (layer "B.Cu") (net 5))
 (segment (start 154.8 118.2) (end 152 121) (width 1) (layer "B.Cu") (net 5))
 (segment (start 144.3 138.6) (end 115.2 138.6) (width 1) (layer "B.Cu") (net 5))
 (segment (start 145.04 102.25) (end 145.04 100.76) (width 1) (layer "B.Cu") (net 5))
 (segment (start 115.2 138.6) (end 110.6 134) (width 1) (layer "B.Cu") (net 5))
 (segment (start 120.8 59.4) (end 120.8 61.6) (width 1) (layer "F.Cu") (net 11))
 (segment (start 161.565 77.035) (end 162.8 75.8) (width 1) (layer "F.Cu") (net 11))
 (segment (start 121.4 58.8) (end 120.8 59.4) (width 1) (layer "F.Cu") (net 11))
 (segment (start 161.025 77.035) (end 161.565 77.035) (width 1) (layer "F.Cu") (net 11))
 (segment (start 148.4 58.8) (end 121.4 58.8) (width 1) (layer "F.Cu") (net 11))
 (segment (start 162.8 73.2) (end 148.4 58.8) (width 1) (layer "F.Cu") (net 11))
 (segment (start 162.8 75.8) (end 162.8 73.2) (width 1) (layer "F.Cu") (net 11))
 (segment (start 120.8 61.6) (end 122.394466 63.194466) (width 1) (layer "F.Cu") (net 11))
 (segment (start 122.394466 63.194466) (end 123.139466 63.194466) (width 1) (layer "F.Cu") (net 11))
 (segment (start 157.475 77.035) (end 155.035 77.035) (width 1) (layer "F.Cu") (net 12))
 (segment (start 155.035 77.035) (end 138.654466 60.654466) (width 1) (layer "F.Cu") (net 12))
 (segment (start 138.654466 60.654466) (end 123.139466 60.654466) (width 1) (layer "F.Cu") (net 12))
 (segment (start 131.935 135.865978) (end 133.200978 134.6) (width 1) (layer "B.Cu") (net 2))
 (segment (start 141.7 134.6) (end 150.12 126.18) (width 1) (layer "B.Cu") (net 2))
 (segment (start 131.935 136.425) (end 131.935 135.865978) (width 1) (layer "B.Cu") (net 2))
 (segment (start 150.12 126.18) (end 150.12 102.25) (width 1) (layer "B.Cu") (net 2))
 (segment (start 133.200978 134.6) (end 141.7 134.6) (width 1) (layer "B.Cu") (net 2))
 (segment (start 146.31 108.6) (end 152.66 102.25) (width 1) (layer "F.Cu") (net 7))
 (segment (start 131.935 132.875) (end 130.940148 131.880148) (width 1) (layer "F.Cu") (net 7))
 (segment (start 130.940148 121.409852) (end 143.75 108.6) (width 1) (layer "F.Cu") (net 7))
 (segment (start 130.940148 131.880148) (end 130.940148 121.409852) (width 1) (layer "F.Cu") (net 7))
 (segment (start 143.75 108.6) (end 146.31 108.6) (width 1) (layer "F.Cu") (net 7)))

